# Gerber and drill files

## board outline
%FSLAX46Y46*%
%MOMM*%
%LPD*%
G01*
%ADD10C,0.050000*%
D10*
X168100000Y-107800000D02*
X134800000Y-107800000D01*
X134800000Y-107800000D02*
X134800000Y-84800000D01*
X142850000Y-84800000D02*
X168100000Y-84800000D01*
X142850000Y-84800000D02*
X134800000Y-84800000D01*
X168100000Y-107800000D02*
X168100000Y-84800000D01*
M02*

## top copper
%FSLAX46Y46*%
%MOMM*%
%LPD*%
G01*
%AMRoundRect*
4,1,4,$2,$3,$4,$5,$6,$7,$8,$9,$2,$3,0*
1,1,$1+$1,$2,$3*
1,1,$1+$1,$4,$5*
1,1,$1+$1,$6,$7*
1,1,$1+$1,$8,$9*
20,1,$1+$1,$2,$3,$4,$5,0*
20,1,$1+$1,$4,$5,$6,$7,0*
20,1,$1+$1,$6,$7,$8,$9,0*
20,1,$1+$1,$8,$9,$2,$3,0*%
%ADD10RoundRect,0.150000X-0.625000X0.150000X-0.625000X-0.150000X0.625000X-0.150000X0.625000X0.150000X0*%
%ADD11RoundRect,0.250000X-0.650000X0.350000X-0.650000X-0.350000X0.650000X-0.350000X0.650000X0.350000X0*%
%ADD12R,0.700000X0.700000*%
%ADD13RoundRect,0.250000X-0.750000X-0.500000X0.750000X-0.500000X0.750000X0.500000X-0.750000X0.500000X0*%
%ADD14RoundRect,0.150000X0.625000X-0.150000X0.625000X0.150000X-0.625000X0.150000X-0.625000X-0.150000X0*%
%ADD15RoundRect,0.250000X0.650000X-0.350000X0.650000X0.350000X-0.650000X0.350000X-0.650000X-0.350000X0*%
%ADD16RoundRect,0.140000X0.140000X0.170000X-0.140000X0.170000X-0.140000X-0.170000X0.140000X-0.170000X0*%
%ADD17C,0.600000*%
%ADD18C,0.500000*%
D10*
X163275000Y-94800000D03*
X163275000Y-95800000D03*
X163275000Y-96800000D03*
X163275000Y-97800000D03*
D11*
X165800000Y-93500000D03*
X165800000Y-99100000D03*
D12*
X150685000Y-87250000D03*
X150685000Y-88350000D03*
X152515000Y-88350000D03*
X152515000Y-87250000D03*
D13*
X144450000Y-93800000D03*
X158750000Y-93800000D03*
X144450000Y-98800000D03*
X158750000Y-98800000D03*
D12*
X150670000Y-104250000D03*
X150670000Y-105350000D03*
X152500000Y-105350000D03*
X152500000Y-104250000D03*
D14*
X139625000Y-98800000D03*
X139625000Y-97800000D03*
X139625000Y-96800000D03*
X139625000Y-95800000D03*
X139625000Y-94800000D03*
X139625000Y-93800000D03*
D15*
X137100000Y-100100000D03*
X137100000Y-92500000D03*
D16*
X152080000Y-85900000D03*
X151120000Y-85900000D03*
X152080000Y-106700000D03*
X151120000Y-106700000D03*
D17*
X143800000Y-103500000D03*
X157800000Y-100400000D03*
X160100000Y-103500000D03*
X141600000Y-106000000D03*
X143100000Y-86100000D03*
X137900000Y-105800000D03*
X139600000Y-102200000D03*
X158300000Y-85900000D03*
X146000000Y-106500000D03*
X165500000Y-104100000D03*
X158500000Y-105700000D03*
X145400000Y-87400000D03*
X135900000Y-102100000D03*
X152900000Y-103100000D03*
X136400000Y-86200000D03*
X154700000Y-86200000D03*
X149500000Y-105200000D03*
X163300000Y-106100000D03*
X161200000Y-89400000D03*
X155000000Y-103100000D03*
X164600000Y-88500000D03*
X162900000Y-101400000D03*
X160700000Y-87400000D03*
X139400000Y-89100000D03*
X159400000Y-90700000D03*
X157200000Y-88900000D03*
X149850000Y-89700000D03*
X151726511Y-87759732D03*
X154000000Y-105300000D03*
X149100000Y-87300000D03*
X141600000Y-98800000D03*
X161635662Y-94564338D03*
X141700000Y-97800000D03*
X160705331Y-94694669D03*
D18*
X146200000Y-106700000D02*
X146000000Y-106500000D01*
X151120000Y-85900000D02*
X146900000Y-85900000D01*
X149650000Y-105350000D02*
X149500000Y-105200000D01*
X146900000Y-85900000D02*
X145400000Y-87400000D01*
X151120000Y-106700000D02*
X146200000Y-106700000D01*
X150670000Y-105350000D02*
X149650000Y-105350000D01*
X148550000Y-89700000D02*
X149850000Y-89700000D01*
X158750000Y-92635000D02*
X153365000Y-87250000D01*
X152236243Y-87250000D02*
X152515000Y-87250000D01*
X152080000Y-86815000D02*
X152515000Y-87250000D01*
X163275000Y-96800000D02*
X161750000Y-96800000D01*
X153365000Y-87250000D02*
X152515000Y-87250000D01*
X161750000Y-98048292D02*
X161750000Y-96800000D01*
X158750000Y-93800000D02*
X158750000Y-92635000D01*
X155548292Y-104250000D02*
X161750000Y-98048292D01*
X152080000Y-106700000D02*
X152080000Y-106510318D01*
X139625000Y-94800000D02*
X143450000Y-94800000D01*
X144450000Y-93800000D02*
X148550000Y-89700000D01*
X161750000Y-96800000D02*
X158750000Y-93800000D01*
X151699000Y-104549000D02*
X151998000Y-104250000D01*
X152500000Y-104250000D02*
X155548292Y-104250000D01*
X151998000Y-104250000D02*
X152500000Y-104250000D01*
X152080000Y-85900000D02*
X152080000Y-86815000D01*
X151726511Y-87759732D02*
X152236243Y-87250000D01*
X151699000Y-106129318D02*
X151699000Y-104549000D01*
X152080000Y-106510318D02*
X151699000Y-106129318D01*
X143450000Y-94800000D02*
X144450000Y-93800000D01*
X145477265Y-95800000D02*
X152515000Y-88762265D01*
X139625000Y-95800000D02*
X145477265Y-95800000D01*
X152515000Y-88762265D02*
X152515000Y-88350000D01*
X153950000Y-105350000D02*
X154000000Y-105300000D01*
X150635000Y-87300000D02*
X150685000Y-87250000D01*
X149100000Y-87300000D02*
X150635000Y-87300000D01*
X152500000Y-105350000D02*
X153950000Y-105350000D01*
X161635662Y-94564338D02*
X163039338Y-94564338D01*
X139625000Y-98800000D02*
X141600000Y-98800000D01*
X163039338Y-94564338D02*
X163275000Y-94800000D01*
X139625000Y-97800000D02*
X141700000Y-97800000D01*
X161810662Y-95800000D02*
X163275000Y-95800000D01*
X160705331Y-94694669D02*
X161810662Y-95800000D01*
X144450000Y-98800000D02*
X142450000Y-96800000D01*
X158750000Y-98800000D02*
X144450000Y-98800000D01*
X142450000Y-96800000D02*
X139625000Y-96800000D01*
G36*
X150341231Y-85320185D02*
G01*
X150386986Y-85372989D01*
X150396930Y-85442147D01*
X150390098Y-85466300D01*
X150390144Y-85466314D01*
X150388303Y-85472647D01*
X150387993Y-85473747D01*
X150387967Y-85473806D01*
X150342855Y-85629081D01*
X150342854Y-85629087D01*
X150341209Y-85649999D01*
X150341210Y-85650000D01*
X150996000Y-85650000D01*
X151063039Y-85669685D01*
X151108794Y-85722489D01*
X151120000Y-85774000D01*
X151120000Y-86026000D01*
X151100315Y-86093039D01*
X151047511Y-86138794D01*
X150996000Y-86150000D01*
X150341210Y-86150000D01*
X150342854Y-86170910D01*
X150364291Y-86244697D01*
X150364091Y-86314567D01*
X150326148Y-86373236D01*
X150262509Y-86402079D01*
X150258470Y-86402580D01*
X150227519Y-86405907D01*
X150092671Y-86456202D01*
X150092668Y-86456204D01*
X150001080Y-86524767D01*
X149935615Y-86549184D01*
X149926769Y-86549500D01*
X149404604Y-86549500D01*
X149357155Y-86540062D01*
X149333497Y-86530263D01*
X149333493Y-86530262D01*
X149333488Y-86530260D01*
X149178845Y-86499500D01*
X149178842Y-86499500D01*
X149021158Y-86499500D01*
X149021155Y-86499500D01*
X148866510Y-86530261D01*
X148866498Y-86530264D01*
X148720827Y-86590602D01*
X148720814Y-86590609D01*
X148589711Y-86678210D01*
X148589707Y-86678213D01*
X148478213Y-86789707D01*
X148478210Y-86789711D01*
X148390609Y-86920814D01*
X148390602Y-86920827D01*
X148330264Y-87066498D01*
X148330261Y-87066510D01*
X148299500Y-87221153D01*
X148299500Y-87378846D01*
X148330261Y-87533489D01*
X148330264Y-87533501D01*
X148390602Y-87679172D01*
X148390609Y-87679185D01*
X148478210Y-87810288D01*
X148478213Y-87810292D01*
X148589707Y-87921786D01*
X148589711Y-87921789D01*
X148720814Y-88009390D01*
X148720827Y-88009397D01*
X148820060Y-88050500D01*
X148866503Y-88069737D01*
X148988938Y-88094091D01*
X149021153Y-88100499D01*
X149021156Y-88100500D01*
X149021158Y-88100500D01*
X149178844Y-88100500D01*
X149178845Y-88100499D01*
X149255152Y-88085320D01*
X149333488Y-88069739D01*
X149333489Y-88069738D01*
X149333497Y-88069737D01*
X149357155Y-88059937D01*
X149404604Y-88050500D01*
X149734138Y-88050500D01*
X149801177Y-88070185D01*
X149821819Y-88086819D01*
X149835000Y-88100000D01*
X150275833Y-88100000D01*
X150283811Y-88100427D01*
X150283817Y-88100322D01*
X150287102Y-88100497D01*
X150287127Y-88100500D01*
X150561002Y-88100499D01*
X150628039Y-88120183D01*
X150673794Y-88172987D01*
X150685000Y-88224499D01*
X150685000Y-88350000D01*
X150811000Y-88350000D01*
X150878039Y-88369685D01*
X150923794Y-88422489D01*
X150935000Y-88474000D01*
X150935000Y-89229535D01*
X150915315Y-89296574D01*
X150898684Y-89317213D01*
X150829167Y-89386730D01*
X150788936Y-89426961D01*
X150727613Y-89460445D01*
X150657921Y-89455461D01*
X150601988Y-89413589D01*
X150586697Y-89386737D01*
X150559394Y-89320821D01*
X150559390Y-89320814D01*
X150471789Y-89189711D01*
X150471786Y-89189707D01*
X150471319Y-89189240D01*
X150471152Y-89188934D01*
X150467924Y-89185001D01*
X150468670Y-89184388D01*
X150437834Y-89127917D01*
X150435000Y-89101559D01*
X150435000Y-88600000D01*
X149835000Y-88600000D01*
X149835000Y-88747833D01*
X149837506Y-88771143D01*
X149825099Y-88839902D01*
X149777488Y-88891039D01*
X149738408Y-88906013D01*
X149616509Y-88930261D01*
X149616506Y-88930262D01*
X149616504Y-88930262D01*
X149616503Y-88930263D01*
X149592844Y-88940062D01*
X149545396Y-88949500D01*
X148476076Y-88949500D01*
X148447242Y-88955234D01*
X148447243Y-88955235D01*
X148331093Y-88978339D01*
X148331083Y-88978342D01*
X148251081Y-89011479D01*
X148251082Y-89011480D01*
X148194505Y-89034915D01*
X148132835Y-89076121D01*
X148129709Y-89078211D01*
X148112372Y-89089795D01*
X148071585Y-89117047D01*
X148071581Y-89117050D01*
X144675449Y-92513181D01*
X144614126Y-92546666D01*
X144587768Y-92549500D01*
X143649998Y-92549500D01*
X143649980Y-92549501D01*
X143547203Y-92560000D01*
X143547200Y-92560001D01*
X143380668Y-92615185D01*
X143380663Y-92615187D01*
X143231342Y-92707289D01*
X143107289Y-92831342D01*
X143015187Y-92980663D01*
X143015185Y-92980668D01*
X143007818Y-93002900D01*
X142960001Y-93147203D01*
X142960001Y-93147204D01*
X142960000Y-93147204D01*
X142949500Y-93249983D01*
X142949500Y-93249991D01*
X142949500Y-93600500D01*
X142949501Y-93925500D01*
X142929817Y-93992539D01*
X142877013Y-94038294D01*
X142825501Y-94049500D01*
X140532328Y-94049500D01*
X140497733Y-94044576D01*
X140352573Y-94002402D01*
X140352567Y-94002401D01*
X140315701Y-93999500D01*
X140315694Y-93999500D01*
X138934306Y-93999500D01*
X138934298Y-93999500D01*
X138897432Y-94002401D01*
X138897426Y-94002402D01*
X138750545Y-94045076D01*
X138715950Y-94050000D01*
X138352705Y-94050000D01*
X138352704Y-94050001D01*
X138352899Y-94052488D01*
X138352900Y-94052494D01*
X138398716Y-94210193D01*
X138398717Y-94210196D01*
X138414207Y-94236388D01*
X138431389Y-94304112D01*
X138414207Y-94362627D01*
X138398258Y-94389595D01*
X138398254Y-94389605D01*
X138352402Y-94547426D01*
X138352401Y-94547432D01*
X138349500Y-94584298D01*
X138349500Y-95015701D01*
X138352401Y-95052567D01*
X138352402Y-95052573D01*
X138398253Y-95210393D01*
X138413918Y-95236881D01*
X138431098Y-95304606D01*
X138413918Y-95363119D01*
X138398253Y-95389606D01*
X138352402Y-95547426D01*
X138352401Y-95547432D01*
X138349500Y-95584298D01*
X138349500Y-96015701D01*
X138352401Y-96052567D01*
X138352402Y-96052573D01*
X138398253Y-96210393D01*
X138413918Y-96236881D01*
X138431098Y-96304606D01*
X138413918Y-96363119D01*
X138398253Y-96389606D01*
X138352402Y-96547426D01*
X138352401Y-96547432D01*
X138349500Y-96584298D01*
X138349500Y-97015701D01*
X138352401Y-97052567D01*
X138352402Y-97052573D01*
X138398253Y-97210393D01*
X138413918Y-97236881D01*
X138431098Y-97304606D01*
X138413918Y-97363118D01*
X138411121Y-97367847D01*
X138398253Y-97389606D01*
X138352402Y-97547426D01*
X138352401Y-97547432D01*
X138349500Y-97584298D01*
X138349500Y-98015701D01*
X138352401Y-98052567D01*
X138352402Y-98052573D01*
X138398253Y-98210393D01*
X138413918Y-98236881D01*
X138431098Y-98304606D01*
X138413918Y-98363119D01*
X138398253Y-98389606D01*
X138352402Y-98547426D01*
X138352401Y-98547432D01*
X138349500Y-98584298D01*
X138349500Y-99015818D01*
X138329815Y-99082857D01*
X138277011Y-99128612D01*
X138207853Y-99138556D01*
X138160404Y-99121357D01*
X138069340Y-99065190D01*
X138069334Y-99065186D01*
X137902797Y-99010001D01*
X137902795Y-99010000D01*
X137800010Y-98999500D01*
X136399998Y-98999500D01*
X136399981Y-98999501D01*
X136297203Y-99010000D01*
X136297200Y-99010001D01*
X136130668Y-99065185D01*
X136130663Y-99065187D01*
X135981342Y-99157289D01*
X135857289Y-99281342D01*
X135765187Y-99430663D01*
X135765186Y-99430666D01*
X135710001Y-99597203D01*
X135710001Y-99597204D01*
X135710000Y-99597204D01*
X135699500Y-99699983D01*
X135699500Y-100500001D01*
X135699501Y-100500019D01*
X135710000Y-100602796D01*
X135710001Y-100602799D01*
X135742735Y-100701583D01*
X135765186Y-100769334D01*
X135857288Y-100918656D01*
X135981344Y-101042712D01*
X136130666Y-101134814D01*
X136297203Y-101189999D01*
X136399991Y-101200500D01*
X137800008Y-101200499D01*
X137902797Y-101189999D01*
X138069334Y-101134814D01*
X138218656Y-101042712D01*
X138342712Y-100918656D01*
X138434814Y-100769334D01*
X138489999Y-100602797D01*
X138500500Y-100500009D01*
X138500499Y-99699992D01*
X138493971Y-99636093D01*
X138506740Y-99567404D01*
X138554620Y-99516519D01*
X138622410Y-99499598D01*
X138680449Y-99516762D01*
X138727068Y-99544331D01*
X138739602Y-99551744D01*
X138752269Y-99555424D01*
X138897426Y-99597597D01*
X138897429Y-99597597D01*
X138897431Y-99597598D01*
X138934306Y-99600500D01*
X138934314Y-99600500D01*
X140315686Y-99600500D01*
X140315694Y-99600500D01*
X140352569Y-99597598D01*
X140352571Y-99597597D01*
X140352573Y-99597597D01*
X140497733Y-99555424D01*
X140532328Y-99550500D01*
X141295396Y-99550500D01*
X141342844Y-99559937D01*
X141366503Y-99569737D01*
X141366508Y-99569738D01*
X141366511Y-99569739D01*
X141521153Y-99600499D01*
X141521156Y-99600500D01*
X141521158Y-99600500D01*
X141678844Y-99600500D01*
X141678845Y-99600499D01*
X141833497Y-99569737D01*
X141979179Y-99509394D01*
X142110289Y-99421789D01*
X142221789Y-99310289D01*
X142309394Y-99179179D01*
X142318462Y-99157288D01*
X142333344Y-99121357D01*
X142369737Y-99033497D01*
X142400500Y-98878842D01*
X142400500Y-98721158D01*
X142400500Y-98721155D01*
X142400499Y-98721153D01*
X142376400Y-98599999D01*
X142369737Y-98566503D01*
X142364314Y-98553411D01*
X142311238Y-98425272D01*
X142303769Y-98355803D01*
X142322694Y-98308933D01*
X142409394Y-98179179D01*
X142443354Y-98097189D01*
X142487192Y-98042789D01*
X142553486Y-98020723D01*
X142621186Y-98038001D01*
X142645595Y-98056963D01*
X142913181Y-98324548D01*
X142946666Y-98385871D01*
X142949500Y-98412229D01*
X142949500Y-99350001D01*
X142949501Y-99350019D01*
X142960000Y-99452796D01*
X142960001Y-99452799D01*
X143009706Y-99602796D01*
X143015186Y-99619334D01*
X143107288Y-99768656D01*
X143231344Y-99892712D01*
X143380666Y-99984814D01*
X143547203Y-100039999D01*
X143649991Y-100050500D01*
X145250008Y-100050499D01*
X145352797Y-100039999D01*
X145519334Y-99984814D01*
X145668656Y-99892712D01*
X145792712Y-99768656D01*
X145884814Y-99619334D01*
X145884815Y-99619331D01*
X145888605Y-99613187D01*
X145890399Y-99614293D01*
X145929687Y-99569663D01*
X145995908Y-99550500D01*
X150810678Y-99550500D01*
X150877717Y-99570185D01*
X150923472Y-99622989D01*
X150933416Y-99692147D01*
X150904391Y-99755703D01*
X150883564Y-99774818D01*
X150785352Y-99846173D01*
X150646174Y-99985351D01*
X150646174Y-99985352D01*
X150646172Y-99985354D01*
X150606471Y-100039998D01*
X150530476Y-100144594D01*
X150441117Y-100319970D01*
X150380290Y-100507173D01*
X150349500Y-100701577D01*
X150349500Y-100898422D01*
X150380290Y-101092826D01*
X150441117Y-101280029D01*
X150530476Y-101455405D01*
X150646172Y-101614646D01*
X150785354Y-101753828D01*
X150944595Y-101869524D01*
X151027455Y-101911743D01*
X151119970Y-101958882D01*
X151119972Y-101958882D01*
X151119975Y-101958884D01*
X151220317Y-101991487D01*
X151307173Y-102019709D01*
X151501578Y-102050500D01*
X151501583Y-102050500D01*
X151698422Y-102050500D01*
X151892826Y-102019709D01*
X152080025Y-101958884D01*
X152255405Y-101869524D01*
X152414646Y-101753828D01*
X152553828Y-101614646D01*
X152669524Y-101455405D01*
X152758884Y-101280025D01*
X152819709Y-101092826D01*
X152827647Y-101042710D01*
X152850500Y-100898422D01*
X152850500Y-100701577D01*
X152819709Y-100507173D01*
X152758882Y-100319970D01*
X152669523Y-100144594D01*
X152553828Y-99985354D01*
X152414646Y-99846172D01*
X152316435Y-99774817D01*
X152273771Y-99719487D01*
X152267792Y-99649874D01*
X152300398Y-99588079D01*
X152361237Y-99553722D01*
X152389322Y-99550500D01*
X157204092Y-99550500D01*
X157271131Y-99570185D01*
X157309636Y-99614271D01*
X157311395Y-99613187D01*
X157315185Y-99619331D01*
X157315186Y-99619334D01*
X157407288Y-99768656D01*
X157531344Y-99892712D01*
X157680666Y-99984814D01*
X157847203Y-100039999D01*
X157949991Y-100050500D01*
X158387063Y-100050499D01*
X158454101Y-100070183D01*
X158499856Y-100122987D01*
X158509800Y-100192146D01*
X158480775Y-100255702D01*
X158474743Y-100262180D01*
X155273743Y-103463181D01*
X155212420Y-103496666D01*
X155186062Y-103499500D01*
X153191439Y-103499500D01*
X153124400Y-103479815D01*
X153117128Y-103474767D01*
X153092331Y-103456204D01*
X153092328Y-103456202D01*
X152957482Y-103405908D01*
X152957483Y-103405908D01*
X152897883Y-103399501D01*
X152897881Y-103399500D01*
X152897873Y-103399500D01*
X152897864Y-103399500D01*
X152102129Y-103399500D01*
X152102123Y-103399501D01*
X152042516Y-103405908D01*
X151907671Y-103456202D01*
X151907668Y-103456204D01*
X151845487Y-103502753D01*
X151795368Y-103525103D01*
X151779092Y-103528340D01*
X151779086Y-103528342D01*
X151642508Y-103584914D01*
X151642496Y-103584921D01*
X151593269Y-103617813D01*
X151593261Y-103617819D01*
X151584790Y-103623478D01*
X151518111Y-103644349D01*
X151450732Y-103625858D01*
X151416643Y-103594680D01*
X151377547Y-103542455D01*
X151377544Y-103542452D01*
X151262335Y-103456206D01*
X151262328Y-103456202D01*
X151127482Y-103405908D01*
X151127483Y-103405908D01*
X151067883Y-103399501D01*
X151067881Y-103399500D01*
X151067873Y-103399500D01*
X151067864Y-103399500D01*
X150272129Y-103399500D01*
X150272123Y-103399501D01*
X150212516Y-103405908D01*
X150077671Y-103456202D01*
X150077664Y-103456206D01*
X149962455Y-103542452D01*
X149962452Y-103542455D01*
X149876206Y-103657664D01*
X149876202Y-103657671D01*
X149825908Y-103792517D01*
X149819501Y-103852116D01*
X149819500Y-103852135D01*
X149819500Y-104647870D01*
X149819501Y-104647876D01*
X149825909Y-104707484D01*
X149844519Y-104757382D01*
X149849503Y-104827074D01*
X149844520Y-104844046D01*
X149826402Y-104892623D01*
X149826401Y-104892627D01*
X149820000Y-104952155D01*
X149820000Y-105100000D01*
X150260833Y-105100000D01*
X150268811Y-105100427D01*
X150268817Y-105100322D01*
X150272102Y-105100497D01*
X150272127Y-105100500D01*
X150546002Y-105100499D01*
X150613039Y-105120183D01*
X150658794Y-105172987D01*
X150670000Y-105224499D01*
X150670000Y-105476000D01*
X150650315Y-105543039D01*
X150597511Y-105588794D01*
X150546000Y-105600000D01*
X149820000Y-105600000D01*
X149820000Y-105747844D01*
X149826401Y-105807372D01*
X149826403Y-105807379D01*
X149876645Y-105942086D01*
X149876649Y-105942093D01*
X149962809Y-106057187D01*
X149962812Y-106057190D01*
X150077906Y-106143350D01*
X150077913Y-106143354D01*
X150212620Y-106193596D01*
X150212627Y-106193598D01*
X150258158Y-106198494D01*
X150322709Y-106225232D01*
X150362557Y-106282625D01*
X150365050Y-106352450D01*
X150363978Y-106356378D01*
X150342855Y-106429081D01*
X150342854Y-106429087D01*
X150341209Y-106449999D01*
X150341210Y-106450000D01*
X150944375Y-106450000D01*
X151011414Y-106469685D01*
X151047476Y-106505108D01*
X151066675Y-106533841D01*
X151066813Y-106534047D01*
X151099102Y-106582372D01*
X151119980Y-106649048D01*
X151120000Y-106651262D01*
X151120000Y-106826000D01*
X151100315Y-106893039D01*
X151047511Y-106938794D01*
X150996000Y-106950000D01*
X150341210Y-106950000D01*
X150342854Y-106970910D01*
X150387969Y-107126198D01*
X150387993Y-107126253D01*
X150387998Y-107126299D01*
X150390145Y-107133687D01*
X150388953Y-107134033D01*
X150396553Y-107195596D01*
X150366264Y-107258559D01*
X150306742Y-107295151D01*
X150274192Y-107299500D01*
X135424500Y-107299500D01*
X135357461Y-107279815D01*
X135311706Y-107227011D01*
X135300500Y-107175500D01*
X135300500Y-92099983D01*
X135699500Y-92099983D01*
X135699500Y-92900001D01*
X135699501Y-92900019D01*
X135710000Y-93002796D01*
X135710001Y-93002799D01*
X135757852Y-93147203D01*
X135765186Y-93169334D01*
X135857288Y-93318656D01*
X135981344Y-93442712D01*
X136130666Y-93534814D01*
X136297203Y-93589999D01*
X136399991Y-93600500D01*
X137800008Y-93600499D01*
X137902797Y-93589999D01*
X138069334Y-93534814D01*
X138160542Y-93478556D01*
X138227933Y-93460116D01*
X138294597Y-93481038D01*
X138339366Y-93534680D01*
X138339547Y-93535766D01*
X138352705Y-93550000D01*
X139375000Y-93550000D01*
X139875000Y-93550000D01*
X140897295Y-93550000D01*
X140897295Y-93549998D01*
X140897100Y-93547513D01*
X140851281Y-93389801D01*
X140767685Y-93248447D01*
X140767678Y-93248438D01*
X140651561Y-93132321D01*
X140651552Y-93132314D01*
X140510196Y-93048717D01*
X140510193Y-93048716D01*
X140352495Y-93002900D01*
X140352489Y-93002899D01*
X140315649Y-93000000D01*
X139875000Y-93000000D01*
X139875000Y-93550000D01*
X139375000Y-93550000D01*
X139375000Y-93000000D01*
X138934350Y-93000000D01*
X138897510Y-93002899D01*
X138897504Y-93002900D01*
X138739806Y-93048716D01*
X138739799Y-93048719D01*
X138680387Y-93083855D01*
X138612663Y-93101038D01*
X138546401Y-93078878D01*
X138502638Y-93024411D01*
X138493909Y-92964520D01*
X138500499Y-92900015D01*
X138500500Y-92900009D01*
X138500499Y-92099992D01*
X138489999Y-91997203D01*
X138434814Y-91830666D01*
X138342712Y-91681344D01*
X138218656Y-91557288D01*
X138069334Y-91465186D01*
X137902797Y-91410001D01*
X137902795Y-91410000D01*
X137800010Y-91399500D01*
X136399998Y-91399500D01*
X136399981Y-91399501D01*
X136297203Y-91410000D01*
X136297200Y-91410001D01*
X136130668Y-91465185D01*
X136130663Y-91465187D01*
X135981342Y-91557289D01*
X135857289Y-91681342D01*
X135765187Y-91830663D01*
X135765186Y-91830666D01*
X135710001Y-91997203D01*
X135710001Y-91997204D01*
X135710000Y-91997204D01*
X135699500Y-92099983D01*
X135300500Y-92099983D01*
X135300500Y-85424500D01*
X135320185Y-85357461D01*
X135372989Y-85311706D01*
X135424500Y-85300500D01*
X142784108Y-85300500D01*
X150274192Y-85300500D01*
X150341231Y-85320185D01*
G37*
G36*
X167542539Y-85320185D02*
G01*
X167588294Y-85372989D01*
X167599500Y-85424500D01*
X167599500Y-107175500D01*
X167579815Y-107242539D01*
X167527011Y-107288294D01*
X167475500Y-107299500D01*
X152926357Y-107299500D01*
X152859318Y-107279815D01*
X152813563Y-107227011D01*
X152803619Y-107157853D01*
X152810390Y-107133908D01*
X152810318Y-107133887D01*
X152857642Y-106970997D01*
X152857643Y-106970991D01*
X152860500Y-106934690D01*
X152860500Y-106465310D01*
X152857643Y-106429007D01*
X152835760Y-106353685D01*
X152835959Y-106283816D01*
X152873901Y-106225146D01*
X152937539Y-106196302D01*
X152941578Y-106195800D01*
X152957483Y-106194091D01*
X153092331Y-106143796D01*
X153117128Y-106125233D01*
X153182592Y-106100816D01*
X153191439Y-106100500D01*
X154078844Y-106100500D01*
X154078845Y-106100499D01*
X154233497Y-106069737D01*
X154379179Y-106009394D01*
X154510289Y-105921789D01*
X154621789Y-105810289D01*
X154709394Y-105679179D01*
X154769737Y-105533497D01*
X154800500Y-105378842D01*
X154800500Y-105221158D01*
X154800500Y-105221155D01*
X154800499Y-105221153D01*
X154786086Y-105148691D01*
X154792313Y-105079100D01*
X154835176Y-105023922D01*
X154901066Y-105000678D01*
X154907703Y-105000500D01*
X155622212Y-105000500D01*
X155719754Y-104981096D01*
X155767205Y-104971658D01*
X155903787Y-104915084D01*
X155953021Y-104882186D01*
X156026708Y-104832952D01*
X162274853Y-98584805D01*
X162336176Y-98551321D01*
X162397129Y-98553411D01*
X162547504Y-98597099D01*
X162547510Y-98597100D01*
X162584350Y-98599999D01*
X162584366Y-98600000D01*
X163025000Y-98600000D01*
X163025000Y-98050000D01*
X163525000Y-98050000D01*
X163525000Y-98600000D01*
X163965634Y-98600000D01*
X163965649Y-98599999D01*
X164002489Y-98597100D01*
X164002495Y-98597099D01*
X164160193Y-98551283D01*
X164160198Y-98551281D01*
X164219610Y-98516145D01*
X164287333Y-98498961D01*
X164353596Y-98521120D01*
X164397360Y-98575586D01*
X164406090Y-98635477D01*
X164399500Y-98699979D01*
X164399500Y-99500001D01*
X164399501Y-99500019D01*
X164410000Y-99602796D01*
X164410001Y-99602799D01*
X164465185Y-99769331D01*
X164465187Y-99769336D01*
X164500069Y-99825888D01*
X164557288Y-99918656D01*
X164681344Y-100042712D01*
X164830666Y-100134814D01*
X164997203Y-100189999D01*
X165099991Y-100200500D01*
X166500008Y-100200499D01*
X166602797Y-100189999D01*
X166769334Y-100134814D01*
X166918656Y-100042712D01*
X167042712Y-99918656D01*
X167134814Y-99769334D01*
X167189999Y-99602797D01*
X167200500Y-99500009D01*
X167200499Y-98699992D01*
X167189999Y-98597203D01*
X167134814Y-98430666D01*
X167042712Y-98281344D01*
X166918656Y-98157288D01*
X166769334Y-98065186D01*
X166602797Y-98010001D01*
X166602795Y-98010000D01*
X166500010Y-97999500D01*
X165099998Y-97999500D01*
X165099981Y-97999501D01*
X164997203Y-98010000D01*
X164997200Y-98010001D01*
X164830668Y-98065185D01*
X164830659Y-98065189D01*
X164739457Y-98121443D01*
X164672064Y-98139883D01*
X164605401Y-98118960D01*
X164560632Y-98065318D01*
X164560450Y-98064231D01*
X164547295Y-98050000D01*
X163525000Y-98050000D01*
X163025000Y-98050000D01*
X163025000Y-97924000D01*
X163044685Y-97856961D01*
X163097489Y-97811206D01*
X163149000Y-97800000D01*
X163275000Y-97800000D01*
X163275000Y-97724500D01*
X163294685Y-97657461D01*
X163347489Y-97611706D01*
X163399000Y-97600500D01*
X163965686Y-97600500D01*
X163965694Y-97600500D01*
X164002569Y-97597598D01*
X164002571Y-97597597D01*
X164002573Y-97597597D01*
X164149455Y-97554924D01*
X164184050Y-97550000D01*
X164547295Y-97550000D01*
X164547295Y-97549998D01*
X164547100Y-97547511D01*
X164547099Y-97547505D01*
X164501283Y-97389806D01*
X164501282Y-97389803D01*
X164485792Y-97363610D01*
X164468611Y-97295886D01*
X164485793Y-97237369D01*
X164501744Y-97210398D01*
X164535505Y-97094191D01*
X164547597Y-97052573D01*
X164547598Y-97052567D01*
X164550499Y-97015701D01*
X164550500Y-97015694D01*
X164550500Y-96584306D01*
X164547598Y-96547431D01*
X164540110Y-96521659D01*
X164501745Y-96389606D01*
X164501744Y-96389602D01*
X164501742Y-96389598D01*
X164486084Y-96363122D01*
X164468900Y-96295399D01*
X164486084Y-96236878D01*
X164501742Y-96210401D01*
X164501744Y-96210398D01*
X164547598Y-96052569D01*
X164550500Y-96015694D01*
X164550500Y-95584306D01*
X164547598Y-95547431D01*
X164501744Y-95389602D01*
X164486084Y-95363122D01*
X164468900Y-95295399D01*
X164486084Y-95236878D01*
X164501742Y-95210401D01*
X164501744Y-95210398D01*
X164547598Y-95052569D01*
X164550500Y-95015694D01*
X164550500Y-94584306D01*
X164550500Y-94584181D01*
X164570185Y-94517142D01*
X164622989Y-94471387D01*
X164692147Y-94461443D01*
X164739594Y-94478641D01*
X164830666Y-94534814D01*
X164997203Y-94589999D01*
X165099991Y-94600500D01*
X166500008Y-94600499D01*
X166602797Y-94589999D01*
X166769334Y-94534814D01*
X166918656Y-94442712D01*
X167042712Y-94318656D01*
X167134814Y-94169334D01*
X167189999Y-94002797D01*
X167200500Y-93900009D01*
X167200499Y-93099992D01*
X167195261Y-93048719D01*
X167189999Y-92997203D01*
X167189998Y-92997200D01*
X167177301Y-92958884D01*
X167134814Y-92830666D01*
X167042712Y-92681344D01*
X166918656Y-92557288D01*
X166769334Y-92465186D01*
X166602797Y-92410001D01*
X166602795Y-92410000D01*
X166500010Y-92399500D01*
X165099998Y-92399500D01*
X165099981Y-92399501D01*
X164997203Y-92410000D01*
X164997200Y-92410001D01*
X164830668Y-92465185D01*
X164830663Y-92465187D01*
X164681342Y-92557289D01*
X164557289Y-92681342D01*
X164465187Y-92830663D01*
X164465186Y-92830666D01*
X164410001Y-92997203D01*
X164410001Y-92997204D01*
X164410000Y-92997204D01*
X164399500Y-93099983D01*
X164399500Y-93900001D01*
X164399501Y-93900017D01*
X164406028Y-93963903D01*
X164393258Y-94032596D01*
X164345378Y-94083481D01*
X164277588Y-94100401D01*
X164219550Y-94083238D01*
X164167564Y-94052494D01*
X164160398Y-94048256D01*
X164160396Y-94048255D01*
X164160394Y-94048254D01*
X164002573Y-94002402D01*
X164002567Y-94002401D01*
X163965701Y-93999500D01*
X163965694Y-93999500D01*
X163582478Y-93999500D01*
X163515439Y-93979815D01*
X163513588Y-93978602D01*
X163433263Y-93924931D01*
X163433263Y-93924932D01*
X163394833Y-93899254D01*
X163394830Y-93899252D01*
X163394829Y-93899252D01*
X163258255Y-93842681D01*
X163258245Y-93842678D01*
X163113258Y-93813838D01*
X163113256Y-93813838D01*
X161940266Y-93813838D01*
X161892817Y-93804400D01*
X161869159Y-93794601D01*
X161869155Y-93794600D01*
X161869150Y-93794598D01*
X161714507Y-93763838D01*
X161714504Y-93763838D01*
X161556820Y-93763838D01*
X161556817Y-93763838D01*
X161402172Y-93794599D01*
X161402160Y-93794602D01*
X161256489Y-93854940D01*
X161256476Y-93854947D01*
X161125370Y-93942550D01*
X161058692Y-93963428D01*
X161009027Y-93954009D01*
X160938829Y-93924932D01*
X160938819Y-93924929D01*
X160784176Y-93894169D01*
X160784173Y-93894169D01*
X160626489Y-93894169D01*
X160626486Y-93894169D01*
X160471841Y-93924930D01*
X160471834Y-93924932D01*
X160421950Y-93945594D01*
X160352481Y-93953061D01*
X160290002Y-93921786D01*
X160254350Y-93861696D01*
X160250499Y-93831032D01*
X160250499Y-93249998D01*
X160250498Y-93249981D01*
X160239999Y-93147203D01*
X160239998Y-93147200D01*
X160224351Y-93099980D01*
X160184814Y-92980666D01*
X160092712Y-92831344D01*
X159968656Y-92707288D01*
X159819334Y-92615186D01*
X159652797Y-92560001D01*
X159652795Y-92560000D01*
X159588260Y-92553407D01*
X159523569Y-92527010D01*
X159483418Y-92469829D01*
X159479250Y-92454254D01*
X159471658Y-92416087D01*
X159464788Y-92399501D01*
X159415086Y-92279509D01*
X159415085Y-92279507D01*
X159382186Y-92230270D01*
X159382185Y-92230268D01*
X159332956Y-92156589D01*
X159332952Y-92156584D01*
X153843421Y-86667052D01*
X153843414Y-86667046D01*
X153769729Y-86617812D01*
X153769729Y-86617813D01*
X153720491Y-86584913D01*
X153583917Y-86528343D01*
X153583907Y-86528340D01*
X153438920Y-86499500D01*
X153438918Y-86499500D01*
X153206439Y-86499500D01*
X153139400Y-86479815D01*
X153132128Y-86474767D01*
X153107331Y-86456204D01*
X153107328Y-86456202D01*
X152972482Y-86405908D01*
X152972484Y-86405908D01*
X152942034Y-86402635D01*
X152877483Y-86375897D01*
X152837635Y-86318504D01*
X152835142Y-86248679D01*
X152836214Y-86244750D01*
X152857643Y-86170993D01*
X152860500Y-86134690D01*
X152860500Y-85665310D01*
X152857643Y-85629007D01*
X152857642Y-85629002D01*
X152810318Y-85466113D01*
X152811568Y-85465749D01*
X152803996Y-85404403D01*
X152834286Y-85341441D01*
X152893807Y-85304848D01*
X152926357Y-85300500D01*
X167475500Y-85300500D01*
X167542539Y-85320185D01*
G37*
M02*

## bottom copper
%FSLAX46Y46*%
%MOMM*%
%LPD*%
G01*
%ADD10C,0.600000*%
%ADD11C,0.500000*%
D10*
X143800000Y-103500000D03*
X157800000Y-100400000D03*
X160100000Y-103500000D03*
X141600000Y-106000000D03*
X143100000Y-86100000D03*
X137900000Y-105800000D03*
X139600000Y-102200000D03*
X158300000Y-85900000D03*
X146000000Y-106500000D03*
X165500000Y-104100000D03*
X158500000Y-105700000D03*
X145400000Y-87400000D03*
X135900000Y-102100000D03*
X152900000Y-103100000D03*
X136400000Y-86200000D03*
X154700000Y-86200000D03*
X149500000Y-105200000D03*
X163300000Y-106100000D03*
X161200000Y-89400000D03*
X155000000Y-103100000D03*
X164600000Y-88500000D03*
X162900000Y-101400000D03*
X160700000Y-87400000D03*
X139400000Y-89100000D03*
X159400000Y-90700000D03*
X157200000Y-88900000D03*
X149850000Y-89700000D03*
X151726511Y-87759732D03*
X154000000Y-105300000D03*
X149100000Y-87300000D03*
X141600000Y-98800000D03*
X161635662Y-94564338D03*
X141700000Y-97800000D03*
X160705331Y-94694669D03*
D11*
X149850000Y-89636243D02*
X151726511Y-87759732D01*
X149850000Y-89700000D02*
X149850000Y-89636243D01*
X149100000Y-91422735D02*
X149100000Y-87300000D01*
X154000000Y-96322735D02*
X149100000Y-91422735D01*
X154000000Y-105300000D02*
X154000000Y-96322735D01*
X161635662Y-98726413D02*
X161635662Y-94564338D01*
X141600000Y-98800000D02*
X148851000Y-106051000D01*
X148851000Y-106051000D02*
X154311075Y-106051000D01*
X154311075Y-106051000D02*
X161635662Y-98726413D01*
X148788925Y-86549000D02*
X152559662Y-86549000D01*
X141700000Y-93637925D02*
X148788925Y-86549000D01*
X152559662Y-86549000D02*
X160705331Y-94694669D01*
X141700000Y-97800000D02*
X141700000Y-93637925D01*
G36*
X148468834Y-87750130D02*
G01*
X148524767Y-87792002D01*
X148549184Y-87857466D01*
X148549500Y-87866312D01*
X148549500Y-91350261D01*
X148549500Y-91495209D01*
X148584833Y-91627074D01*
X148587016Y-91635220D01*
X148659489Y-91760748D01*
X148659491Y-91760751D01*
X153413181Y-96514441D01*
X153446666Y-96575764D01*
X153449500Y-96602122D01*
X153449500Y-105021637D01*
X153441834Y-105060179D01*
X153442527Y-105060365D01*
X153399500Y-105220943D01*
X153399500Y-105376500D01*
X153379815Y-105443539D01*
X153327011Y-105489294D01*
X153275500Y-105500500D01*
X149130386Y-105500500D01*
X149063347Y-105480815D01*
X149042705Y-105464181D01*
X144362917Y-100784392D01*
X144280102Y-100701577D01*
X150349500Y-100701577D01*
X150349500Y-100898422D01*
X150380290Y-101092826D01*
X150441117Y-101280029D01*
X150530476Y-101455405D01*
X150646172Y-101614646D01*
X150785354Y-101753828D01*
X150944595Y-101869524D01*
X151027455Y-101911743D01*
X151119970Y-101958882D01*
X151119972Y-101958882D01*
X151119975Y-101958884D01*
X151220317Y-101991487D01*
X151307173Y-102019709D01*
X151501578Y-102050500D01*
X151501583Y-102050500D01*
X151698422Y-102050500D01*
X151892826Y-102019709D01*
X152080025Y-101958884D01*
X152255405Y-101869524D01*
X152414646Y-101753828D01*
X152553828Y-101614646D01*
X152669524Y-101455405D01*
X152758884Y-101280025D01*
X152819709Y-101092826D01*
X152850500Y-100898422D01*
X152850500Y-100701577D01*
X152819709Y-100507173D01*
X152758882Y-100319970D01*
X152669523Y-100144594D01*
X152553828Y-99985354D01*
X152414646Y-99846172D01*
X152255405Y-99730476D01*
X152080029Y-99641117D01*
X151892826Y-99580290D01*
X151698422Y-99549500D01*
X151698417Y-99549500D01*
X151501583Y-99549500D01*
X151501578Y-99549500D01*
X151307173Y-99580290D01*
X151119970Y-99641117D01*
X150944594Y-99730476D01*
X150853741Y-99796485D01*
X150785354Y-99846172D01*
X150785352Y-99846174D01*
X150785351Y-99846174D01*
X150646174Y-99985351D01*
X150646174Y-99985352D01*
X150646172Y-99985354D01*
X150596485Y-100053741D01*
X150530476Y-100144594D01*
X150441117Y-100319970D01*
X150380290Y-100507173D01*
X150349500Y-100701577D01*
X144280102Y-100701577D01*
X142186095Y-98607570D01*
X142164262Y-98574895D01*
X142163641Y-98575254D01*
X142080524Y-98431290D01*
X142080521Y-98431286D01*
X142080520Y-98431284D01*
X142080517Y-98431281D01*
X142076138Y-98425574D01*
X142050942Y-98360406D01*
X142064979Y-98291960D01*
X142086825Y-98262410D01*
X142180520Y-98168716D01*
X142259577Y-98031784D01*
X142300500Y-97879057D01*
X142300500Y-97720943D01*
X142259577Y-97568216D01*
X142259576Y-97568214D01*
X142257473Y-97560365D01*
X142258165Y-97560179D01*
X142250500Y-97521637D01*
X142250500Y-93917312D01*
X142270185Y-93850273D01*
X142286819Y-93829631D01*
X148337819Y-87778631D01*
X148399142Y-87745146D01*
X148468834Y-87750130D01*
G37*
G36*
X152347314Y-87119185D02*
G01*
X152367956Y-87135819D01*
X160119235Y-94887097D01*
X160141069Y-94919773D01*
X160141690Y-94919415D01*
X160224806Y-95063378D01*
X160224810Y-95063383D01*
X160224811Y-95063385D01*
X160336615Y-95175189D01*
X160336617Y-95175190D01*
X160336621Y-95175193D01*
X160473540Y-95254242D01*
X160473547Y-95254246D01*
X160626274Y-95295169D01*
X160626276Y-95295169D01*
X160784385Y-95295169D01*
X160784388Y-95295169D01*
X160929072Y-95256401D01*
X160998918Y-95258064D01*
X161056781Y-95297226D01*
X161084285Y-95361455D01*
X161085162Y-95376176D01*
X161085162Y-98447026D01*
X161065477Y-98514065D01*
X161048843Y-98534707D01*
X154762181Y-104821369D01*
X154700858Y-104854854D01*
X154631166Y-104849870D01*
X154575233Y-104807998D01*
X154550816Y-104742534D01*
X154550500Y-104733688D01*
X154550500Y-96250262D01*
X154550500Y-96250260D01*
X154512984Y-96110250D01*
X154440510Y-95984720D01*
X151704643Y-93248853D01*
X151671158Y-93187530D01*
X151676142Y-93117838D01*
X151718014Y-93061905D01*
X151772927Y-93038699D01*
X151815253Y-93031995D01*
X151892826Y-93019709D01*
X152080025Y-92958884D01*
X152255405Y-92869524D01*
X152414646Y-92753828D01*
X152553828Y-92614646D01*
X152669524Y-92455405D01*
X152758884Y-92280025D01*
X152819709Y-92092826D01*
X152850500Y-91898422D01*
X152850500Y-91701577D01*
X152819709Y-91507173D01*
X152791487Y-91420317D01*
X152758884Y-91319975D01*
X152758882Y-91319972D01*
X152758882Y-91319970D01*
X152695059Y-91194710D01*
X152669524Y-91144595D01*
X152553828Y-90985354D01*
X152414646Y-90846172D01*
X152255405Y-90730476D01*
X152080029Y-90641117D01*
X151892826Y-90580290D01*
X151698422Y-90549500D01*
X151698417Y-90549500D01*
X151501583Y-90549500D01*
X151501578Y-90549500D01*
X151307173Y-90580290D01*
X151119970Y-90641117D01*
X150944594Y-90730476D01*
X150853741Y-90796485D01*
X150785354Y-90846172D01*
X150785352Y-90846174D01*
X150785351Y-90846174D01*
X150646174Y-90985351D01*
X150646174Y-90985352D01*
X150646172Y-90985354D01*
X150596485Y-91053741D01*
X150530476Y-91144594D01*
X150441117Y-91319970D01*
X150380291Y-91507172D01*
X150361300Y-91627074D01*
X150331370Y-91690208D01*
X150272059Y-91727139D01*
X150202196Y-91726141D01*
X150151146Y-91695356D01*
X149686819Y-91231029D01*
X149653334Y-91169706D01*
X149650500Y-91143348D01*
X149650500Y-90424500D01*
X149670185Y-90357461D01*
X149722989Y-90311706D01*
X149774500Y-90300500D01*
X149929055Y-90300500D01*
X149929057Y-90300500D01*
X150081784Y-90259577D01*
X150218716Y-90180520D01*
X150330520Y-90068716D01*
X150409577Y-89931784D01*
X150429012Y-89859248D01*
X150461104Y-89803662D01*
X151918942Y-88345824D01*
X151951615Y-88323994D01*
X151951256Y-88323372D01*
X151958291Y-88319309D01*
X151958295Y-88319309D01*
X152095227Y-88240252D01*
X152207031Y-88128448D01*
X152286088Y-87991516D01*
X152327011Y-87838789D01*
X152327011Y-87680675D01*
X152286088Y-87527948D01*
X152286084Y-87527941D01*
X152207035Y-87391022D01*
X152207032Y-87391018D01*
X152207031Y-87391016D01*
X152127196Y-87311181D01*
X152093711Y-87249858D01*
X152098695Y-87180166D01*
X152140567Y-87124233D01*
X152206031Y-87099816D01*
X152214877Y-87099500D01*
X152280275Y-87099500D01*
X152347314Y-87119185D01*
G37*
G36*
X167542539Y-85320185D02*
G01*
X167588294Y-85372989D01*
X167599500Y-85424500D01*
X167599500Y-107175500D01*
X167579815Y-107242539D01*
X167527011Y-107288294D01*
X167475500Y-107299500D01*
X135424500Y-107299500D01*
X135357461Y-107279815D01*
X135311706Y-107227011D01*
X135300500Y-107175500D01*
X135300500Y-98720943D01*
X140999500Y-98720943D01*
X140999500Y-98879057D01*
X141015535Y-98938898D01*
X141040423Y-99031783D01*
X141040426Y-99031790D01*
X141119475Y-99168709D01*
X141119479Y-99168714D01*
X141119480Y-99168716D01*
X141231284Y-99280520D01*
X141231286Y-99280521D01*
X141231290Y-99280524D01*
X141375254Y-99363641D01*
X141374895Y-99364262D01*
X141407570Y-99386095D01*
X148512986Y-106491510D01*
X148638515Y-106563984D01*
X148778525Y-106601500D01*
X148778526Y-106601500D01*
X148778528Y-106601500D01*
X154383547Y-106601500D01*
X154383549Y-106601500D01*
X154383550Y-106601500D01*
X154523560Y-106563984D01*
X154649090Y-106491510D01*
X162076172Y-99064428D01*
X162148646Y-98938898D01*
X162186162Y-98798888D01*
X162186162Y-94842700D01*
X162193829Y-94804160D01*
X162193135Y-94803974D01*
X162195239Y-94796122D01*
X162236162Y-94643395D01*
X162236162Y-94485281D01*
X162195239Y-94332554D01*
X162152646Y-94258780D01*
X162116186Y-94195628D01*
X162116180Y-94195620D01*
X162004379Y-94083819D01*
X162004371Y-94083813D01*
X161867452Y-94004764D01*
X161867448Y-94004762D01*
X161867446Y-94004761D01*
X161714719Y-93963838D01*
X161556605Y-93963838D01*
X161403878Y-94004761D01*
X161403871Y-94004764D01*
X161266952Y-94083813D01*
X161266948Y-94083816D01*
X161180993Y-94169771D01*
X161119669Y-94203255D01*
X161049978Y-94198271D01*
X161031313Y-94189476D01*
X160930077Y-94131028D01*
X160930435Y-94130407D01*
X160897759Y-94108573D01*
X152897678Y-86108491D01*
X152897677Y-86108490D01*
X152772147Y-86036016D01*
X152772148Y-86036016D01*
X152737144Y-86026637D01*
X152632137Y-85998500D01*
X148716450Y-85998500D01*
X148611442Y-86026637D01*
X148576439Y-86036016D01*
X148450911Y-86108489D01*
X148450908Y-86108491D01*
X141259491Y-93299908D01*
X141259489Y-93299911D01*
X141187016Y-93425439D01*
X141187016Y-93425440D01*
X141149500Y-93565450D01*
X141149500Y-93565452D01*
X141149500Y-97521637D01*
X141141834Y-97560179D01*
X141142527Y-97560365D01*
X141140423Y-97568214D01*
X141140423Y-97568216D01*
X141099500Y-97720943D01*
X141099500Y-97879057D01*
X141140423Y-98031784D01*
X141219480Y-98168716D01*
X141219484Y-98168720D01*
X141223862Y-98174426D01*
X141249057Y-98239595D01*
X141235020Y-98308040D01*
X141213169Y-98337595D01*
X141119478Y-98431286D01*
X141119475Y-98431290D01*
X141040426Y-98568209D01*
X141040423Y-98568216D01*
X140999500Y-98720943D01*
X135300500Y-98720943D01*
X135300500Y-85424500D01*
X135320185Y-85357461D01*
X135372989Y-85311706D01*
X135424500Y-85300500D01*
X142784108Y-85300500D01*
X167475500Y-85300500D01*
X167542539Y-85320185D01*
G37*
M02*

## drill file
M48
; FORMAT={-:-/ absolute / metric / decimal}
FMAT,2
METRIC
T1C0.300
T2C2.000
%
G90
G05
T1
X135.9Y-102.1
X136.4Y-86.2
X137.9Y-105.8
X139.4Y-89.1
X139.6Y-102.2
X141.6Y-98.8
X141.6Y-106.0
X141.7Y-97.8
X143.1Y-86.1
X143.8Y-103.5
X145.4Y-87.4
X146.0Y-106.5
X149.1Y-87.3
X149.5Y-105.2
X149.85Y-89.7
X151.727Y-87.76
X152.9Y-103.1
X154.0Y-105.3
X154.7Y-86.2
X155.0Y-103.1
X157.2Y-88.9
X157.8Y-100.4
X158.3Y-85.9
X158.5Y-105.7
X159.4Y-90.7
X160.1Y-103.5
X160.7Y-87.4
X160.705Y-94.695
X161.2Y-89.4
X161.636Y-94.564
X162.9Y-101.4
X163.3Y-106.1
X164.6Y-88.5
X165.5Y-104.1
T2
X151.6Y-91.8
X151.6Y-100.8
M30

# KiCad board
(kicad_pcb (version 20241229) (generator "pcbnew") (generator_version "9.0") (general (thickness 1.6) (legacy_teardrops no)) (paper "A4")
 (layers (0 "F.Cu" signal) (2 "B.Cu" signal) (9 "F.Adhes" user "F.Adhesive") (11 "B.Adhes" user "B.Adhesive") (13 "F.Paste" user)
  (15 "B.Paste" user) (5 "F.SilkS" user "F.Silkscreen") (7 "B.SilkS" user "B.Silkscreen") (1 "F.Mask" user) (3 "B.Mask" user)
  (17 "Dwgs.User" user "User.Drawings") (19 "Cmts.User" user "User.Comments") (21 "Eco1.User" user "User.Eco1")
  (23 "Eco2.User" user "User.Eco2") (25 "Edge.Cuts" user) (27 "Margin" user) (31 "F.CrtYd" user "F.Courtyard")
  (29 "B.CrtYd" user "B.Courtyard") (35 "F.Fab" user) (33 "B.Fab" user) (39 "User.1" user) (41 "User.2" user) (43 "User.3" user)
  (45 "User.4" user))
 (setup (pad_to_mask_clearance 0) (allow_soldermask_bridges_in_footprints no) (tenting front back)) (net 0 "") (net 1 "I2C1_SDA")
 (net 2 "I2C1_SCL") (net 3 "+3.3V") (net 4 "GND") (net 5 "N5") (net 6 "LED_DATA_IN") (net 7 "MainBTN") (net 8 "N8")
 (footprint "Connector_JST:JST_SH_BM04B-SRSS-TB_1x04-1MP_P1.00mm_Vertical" (layer "F.Cu") (at 164.6 96.3 -90)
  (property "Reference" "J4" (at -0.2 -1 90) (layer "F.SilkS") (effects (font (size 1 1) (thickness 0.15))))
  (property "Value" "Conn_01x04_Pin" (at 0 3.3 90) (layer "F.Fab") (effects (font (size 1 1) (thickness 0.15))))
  (pad "1" smd roundrect (at -1.5 1.325 270) (size 0.6 1.55) (layers "F.Cu" "F.Mask" "F.Paste") (roundrect_rratio 0.25) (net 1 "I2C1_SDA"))
  (pad "2" smd roundrect (at -0.5 1.325 270) (size 0.6 1.55) (layers "F.Cu" "F.Mask" "F.Paste") (roundrect_rratio 0.25) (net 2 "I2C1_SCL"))
  (pad "3" smd roundrect (at 0.5 1.325 270) (size 0.6 1.55) (layers "F.Cu" "F.Mask" "F.Paste") (roundrect_rratio 0.25) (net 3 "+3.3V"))
  (pad "4" smd roundrect (at 1.5 1.325 270) (size 0.6 1.55) (layers "F.Cu" "F.Mask" "F.Paste") (roundrect_rratio 0.25) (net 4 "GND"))
  (pad "MP" smd roundrect (at -2.8 -1.2 270) (size 1.2 1.8) (layers "F.Cu" "F.Mask" "F.Paste") (roundrect_rratio 0.208333))
  (pad "MP" smd roundrect (at 2.8 -1.2 270) (size 1.2 1.8) (layers "F.Cu" "F.Mask" "F.Paste") (roundrect_rratio 0.208333)))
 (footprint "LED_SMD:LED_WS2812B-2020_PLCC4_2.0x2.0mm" (layer "F.Cu") (at 151.6 87.8)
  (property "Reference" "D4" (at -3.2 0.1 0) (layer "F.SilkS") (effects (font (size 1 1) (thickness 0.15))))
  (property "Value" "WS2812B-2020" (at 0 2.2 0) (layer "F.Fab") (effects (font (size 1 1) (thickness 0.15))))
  (pad "1" smd rect (at -0.915 -0.55) (size 0.7 0.7) (layers "F.Cu" "F.Mask" "F.Paste") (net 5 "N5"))
  (pad "2" smd rect (at -0.915 0.55) (size 0.7 0.7) (layers "F.Cu" "F.Mask" "F.Paste") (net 4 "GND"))
  (pad "3" smd rect (at 0.915 0.55) (size 0.7 0.7) (layers "F.Cu" "F.Mask" "F.Paste") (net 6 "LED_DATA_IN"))
  (pad "4" smd rect (at 0.915 -0.55) (size 0.7 0.7) (layers "F.Cu" "F.Mask" "F.Paste") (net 3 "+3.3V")))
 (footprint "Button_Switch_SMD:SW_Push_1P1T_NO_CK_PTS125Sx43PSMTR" (layer "F.Cu") (at 151.6 96.3)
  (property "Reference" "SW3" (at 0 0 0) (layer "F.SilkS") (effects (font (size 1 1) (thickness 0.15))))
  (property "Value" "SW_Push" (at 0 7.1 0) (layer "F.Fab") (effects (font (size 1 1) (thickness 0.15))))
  (pad "" np_thru_hole circle (at 0 -4.5) (size 2 2) (drill 2) (layers "*.Cu" "*.Mask"))
  (pad "" np_thru_hole circle (at 0 4.5) (size 2 2) (drill 2) (layers "*.Cu" "*.Mask"))
  (pad "1" smd roundrect (at -7.15 -2.5) (size 2 1.5) (layers "F.Cu" "F.Mask" "F.Paste") (roundrect_rratio 0.1666666667) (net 3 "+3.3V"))
  (pad "1" smd roundrect (at 7.15 -2.5) (size 2 1.5) (layers "F.Cu" "F.Mask" "F.Paste") (roundrect_rratio 0.1666666667) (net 3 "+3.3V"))
  (pad "2" smd roundrect (at -7.15 2.5) (size 2 1.5) (layers "F.Cu" "F.Mask" "F.Paste") (roundrect_rratio 0.1666666667) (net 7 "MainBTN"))
  (pad "2" smd roundrect (at 7.15 2.5) (size 2 1.5) (layers "F.Cu" "F.Mask" "F.Paste") (roundrect_rratio 0.1666666667) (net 7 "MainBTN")))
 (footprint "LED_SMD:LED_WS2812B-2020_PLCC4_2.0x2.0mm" (layer "F.Cu") (at 151.585 104.8)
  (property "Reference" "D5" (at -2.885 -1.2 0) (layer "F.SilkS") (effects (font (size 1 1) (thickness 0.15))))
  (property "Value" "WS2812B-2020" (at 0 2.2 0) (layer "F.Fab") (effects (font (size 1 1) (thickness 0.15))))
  (pad "1" smd rect (at -0.915 -0.55) (size 0.7 0.7) (layers "F.Cu" "F.Mask" "F.Paste") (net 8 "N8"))
  (pad "2" smd rect (at -0.915 0.55) (size 0.7 0.7) (layers "F.Cu" "F.Mask" "F.Paste") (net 4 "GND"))
  (pad "3" smd rect (at 0.915 0.55) (size 0.7 0.7) (layers "F.Cu" "F.Mask" "F.Paste") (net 5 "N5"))
  (pad "4" smd rect (at 0.915 -0.55) (size 0.7 0.7) (layers "F.Cu" "F.Mask" "F.Paste") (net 3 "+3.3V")))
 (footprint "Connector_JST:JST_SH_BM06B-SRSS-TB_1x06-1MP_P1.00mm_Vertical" (layer "F.Cu") (at 138.3 96.3 90)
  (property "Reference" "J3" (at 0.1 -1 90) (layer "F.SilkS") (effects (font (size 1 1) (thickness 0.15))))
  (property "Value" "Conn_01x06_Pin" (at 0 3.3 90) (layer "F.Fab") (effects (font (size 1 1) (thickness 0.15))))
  (pad "1" smd roundrect (at -2.5 1.325 90) (size 0.6 1.55) (layers "F.Cu" "F.Mask" "F.Paste") (roundrect_rratio 0.25) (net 1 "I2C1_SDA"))
  (pad "2" smd roundrect (at -1.5 1.325 90) (size 0.6 1.55) (layers "F.Cu" "F.Mask" "F.Paste") (roundrect_rratio 0.25) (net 2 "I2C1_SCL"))
  (pad "3" smd roundrect (at -0.5 1.325 90) (size 0.6 1.55) (layers "F.Cu" "F.Mask" "F.Paste") (roundrect_rratio 0.25) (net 7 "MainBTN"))
  (pad "4" smd roundrect (at 0.5 1.325 90) (size 0.6 1.55) (layers "F.Cu" "F.Mask" "F.Paste") (roundrect_rratio 0.25) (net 6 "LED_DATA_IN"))
  (pad "5" smd roundrect (at 1.5 1.325 90) (size 0.6 1.55) (layers "F.Cu" "F.Mask" "F.Paste") (roundrect_rratio 0.25) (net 3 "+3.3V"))
  (pad "6" smd roundrect (at 2.5 1.325 90) (size 0.6 1.55) (layers "F.Cu" "F.Mask" "F.Paste") (roundrect_rratio 0.25) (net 4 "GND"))
  (pad "MP" smd roundrect (at -3.8 -1.2 90) (size 1.2 1.8) (layers "F.Cu" "F.Mask" "F.Paste") (roundrect_rratio 0.208333))
  (pad "MP" smd roundrect (at 3.8 -1.2 90) (size 1.2 1.8) (layers "F.Cu" "F.Mask" "F.Paste") (roundrect_rratio 0.208333)))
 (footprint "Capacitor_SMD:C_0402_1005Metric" (layer "F.Cu") (at 151.6 85.9 180)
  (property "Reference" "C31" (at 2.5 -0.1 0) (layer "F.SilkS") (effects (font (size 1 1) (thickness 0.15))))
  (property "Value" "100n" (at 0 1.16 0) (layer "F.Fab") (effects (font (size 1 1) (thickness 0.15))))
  (pad "1" smd roundrect (at -0.48 0 180) (size 0.56 0.62) (layers "F.Cu" "F.Mask" "F.Paste") (roundrect_rratio 0.25) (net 3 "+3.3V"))
  (pad "2" smd roundrect (at 0.48 0 180) (size 0.56 0.62) (layers "F.Cu" "F.Mask" "F.Paste") (roundrect_rratio 0.25) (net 4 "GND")))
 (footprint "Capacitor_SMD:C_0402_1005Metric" (layer "F.Cu") (at 151.6 106.7 180)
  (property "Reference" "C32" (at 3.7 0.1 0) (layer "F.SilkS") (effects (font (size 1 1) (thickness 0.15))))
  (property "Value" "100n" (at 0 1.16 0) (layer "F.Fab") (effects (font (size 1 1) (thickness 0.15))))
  (pad "1" smd roundrect (at -0.48 0 180) (size 0.56 0.62) (layers "F.Cu" "F.Mask" "F.Paste") (roundrect_rratio 0.25) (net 3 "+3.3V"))
  (pad "2" smd roundrect (at 0.48 0 180) (size 0.56 0.62) (layers "F.Cu" "F.Mask" "F.Paste") (roundrect_rratio 0.25) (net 4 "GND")))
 (gr_line (start 168.1 107.8) (end 134.8 107.8) (stroke (width 0.05) (type default)) (layer "Edge.Cuts"))
 (gr_line (start 134.8 107.8) (end 134.8 84.8) (stroke (width 0.05) (type default)) (layer "Edge.Cuts"))
 (gr_line (start 142.85 84.8) (end 168.1 84.8) (stroke (width 0.05) (type default)) (layer "Edge.Cuts"))
 (gr_line (start 142.85 84.8) (end 134.8 84.8) (stroke (width 0.05) (type default)) (layer "Edge.Cuts"))
 (gr_line (start 168.1 107.8) (end 168.1 84.8) (stroke (width 0.05) (type default)) (layer "Edge.Cuts"))
 (segment (start 146.2 106.7) (end 146 106.5) (width 0.5) (layer "F.Cu") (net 4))
 (segment (start 151.12 85.9) (end 146.9 85.9) (width 0.5) (layer "F.Cu") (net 4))
 (segment (start 149.65 105.35) (end 149.5 105.2) (width 0.5) (layer "F.Cu") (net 4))
 (segment (start 146.9 85.9) (end 145.4 87.4) (width 0.5) (layer "F.Cu") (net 4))
 (segment (start 151.12 106.7) (end 146.2 106.7) (width 0.5) (layer "F.Cu") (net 4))
 (segment (start 150.67 105.35) (end 149.65 105.35) (width 0.5) (layer "F.Cu") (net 4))
 (via (at 143.8 103.5) (size 0.6) (drill 0.3) (layers "F.Cu" "B.Cu") (free yes) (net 4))
 (via (at 157.8 100.4) (size 0.6) (drill 0.3) (layers "F.Cu" "B.Cu") (free yes) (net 4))
 (via (at 160.1 103.5) (size 0.6) (drill 0.3) (layers "F.Cu" "B.Cu") (free yes) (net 4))
 (via (at 141.6 106) (size 0.6) (drill 0.3) (layers "F.Cu" "B.Cu") (free yes) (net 4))
 (via (at 143.1 86.1) (size 0.6) (drill 0.3) (layers "F.Cu" "B.Cu") (free yes) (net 4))
 (via (at 137.9 105.8) (size 0.6) (drill 0.3) (layers "F.Cu" "B.Cu") (free yes) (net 4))
 (via (at 139.6 102.2) (size 0.6) (drill 0.3) (layers "F.Cu" "B.Cu") (free yes) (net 4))
 (via (at 158.3 85.9) (size 0.6) (drill 0.3) (layers "F.Cu" "B.Cu") (free yes) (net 4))
 (via (at 146 106.5) (size 0.6) (drill 0.3) (layers "F.Cu" "B.Cu") (free yes) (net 4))
 (via (at 165.5 104.1) (size 0.6) (drill 0.3) (layers "F.Cu" "B.Cu") (free yes) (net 4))
 (via (at 158.5 105.7) (size 0.6) (drill 0.3) (layers "F.Cu" "B.Cu") (free yes) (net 4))
 (via (at 145.4 87.4) (size 0.6) (drill 0.3) (layers "F.Cu" "B.Cu") (free yes) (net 4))
 (via (at 135.9 102.1) (size 0.6) (drill 0.3) (layers "F.Cu" "B.Cu") (free yes) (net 4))
 (via (at 152.9 103.1) (size 0.6) (drill 0.3) (layers "F.Cu" "B.Cu") (free yes) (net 4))
 (via (at 136.4 86.2) (size 0.6) (drill 0.3) (layers "F.Cu" "B.Cu") (free yes) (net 4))
 (via (at 154.7 86.2) (size 0.6) (drill 0.3) (layers "F.Cu" "B.Cu") (free yes) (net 4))
 (via (at 149.5 105.2) (size 0.6) (drill 0.3) (layers "F.Cu" "B.Cu") (free yes) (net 4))
 (via (at 163.3 106.1) (size 0.6) (drill 0.3) (layers "F.Cu" "B.Cu") (free yes) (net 4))
 (via (at 161.2 89.4) (size 0.6) (drill 0.3) (layers "F.Cu" "B.Cu") (free yes) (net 4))
 (via (at 155 103.1) (size 0.6) (drill 0.3) (layers "F.Cu" "B.Cu") (free yes) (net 4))
 (via (at 164.6 88.5) (size 0.6) (drill 0.3) (layers "F.Cu" "B.Cu") (free yes) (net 4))
 (via (at 162.9 101.4) (size 0.6) (drill 0.3) (layers "F.Cu" "B.Cu") (free yes) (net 4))
 (via (at 160.7 87.4) (size 0.6) (drill 0.3) (layers "F.Cu" "B.Cu") (free yes) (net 4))
 (via (at 139.4 89.1) (size 0.6) (drill 0.3) (layers "F.Cu" "B.Cu") (free yes) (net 4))
 (via (at 159.4 90.7) (size 0.6) (drill 0.3) (layers "F.Cu" "B.Cu") (free yes) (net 4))
 (via (at 157.2 88.9) (size 0.6) (drill 0.3) (layers "F.Cu" "B.Cu") (free yes) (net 4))
 (segment (start 148.55 89.7) (end 149.85 89.7) (width 0.5) (layer "F.Cu") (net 3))
 (segment (start 158.75 92.635) (end 153.365 87.25) (width 0.5) (layer "F.Cu") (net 3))
 (segment (start 152.236243 87.25) (end 152.515 87.25) (width 0.5) (layer "F.Cu") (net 3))
 (segment (start 152.08 86.815) (end 152.515 87.25) (width 0.5) (layer "F.Cu") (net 3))
 (segment (start 163.275 96.8) (end 161.75 96.8) (width 0.5) (layer "F.Cu") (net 3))
 (segment (start 153.365 87.25) (end 152.515 87.25) (width 0.5) (layer "F.Cu") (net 3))
 (segment (start 161.75 98.048292) (end 161.75 96.8) (width 0.5) (layer "F.Cu") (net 3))
 (segment (start 158.75 93.8) (end 158.75 92.635) (width 0.5) (layer "F.Cu") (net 3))
 (segment (start 155.548292 104.25) (end 161.75 98.048292) (width 0.5) (layer "F.Cu") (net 3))
 (segment (start 152.08 106.7) (end 152.08 106.510318) (width 0.5) (layer "F.Cu") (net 3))
 (segment (start 139.625 94.8) (end 143.45 94.8) (width 0.5) (layer "F.Cu") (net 3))
 (segment (start 144.45 93.8) (end 148.55 89.7) (width 0.5) (layer "F.Cu") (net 3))
 (segment (start 161.75 96.8) (end 158.75 93.8) (width 0.5) (layer "F.Cu") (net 3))
 (segment (start 151.699 104.549) (end 151.998 104.25) (width 0.5) (layer "F.Cu") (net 3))
 (segment (start 152.5 104.25) (end 155.548292 104.25) (width 0.5) (layer "F.Cu") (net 3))
 (segment (start 151.998 104.25) (end 152.5 104.25) (width 0.5) (layer "F.Cu") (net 3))
 (segment (start 152.08 85.9) (end 152.08 86.815) (width 0.5) (layer "F.Cu") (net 3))
 (segment (start 151.726511 87.759732) (end 152.236243 87.25) (width 0.5) (layer "F.Cu") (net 3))
 (segment (start 151.699 106.129318) (end 151.699 104.549) (width 0.5) (layer "F.Cu") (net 3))
 (segment (start 152.08 106.510318) (end 151.699 106.129318) (width 0.5) (layer "F.Cu") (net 3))
 (segment (start 143.45 94.8) (end 144.45 93.8) (width 0.5) (layer "F.Cu") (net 3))
 (via (at 149.85 89.7) (size 0.6) (drill 0.3) (layers "F.Cu" "B.Cu") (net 3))
 (via (at 151.726511 87.759732) (size 0.6) (drill 0.3) (layers "F.Cu" "B.Cu") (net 3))
 (segment (start 149.85 89.636243) (end 151.726511 87.759732) (width 0.5) (layer "B.Cu") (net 3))
 (segment (start 149.85 89.7) (end 149.85 89.636243) (width 0.5) (layer "B.Cu") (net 3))
 (segment (start 145.477265 95.8) (end 152.515 88.762265) (width 0.5) (layer "F.Cu") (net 6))
 (segment (start 139.625 95.8) (end 145.477265 95.8) (width 0.5) (layer "F.Cu") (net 6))
 (segment (start 152.515 88.762265) (end 152.515 88.35) (width 0.5) (layer "F.Cu") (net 6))
 (segment (start 153.95 105.35) (end 154 105.3) (width 0.5) (layer "F.Cu") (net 5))
 (segment (start 150.635 87.3) (end 150.685 87.25) (width 0.5) (layer "F.Cu") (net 5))
 (segment (start 149.1 87.3) (end 150.635 87.3) (width 0.5) (layer "F.Cu") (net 5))
 (segment (start 152.5 105.35) (end 153.95 105.35) (width 0.5) (layer "F.Cu") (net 5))
 (via (at 154 105.3) (size 0.6) (drill 0.3) (layers "F.Cu" "B.Cu") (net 5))
 (via (at 149.1 87.3) (size 0.6) (drill 0.3) (layers "F.Cu" "B.Cu") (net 5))
 (segment (start 149.1 91.422735) (end 149.1 87.3) (width 0.5) (layer "B.Cu") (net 5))
 (segment (start 154 96.322735) (end 149.1 91.422735) (width 0.5) (layer "B.Cu") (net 5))
 (segment (start 154 105.3) (end 154 96.322735) (width 0.5) (layer "B.Cu") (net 5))
 (segment (start 161.635662 94.564338) (end 163.039338 94.564338) (width 0.5) (layer "F.Cu") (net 1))
 (segment (start 139.625 98.8) (end 141.6 98.8) (width 0.5) (layer "F.Cu") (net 1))
 (segment (start 163.039338 94.564338) (end 163.275 94.8) (width 0.5) (layer "F.Cu") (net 1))
 (via (at 141.6 98.8) (size 0.6) (drill 0.3) (layers "F.Cu" "B.Cu") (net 1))
 (via (at 161.635662 94.564338) (size 0.6) (drill 0.3) (layers "F.Cu" "B.Cu") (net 1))
 (segment (start 161.635662 98.726413) (end 161.635662 94.564338) (width 0.5) (layer "B.Cu") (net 1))
 (segment (start 141.6 98.8) (end 148.851 106.051) (width 0.5) (layer "B.Cu") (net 1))
 (segment (start 148.851 106.051) (end 154.311075 106.051) (width 0.5) (layer "B.Cu") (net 1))
 (segment (start 154.311075 106.051) (end 161.635662 98.726413) (width 0.5) (layer "B.Cu") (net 1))
 (segment (start 139.625 97.8) (end 141.7 97.8) (width 0.5) (layer "F.Cu") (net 2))
 (segment (start 161.810662 95.8) (end 163.275 95.8) (width 0.5) (layer "F.Cu") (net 2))
 (segment (start 160.705331 94.694669) (end 161.810662 95.8) (width 0.5) (layer "F.Cu") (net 2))
 (via (at 141.7 97.8) (size 0.6) (drill 0.3) (layers "F.Cu" "B.Cu") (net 2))
 (via (at 160.705331 94.694669) (size 0.6) (drill 0.3) (layers "F.Cu" "B.Cu") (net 2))
 (segment (start 148.788925 86.549) (end 152.559662 86.549) (width 0.5) (layer "B.Cu") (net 2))
 (segment (start 141.7 93.637925) (end 148.788925 86.549) (width 0.5) (layer "B.Cu") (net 2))
 (segment (start 152.559662 86.549) (end 160.705331 94.694669) (width 0.5) (layer "B.Cu") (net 2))
 (segment (start 141.7 97.8) (end 141.7 93.637925) (width 0.5) (layer "B.Cu") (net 2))
 (segment (start 144.45 98.8) (end 142.45 96.8) (width 0.5) (layer "F.Cu") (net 7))
 (segment (start 158.75 98.8) (end 144.45 98.8) (width 0.5) (layer "F.Cu") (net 7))
 (segment (start 142.45 96.8) (end 139.625 96.8) (width 0.5) (layer "F.Cu") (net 7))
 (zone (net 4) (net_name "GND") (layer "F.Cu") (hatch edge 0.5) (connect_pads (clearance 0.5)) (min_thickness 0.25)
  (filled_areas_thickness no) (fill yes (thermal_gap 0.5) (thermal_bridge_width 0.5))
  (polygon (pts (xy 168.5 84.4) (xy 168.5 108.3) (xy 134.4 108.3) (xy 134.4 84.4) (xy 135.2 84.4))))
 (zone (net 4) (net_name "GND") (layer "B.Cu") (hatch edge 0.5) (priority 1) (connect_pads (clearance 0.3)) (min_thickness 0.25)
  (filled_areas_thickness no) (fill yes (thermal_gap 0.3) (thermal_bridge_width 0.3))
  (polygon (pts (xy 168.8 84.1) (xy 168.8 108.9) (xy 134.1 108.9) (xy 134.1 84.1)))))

